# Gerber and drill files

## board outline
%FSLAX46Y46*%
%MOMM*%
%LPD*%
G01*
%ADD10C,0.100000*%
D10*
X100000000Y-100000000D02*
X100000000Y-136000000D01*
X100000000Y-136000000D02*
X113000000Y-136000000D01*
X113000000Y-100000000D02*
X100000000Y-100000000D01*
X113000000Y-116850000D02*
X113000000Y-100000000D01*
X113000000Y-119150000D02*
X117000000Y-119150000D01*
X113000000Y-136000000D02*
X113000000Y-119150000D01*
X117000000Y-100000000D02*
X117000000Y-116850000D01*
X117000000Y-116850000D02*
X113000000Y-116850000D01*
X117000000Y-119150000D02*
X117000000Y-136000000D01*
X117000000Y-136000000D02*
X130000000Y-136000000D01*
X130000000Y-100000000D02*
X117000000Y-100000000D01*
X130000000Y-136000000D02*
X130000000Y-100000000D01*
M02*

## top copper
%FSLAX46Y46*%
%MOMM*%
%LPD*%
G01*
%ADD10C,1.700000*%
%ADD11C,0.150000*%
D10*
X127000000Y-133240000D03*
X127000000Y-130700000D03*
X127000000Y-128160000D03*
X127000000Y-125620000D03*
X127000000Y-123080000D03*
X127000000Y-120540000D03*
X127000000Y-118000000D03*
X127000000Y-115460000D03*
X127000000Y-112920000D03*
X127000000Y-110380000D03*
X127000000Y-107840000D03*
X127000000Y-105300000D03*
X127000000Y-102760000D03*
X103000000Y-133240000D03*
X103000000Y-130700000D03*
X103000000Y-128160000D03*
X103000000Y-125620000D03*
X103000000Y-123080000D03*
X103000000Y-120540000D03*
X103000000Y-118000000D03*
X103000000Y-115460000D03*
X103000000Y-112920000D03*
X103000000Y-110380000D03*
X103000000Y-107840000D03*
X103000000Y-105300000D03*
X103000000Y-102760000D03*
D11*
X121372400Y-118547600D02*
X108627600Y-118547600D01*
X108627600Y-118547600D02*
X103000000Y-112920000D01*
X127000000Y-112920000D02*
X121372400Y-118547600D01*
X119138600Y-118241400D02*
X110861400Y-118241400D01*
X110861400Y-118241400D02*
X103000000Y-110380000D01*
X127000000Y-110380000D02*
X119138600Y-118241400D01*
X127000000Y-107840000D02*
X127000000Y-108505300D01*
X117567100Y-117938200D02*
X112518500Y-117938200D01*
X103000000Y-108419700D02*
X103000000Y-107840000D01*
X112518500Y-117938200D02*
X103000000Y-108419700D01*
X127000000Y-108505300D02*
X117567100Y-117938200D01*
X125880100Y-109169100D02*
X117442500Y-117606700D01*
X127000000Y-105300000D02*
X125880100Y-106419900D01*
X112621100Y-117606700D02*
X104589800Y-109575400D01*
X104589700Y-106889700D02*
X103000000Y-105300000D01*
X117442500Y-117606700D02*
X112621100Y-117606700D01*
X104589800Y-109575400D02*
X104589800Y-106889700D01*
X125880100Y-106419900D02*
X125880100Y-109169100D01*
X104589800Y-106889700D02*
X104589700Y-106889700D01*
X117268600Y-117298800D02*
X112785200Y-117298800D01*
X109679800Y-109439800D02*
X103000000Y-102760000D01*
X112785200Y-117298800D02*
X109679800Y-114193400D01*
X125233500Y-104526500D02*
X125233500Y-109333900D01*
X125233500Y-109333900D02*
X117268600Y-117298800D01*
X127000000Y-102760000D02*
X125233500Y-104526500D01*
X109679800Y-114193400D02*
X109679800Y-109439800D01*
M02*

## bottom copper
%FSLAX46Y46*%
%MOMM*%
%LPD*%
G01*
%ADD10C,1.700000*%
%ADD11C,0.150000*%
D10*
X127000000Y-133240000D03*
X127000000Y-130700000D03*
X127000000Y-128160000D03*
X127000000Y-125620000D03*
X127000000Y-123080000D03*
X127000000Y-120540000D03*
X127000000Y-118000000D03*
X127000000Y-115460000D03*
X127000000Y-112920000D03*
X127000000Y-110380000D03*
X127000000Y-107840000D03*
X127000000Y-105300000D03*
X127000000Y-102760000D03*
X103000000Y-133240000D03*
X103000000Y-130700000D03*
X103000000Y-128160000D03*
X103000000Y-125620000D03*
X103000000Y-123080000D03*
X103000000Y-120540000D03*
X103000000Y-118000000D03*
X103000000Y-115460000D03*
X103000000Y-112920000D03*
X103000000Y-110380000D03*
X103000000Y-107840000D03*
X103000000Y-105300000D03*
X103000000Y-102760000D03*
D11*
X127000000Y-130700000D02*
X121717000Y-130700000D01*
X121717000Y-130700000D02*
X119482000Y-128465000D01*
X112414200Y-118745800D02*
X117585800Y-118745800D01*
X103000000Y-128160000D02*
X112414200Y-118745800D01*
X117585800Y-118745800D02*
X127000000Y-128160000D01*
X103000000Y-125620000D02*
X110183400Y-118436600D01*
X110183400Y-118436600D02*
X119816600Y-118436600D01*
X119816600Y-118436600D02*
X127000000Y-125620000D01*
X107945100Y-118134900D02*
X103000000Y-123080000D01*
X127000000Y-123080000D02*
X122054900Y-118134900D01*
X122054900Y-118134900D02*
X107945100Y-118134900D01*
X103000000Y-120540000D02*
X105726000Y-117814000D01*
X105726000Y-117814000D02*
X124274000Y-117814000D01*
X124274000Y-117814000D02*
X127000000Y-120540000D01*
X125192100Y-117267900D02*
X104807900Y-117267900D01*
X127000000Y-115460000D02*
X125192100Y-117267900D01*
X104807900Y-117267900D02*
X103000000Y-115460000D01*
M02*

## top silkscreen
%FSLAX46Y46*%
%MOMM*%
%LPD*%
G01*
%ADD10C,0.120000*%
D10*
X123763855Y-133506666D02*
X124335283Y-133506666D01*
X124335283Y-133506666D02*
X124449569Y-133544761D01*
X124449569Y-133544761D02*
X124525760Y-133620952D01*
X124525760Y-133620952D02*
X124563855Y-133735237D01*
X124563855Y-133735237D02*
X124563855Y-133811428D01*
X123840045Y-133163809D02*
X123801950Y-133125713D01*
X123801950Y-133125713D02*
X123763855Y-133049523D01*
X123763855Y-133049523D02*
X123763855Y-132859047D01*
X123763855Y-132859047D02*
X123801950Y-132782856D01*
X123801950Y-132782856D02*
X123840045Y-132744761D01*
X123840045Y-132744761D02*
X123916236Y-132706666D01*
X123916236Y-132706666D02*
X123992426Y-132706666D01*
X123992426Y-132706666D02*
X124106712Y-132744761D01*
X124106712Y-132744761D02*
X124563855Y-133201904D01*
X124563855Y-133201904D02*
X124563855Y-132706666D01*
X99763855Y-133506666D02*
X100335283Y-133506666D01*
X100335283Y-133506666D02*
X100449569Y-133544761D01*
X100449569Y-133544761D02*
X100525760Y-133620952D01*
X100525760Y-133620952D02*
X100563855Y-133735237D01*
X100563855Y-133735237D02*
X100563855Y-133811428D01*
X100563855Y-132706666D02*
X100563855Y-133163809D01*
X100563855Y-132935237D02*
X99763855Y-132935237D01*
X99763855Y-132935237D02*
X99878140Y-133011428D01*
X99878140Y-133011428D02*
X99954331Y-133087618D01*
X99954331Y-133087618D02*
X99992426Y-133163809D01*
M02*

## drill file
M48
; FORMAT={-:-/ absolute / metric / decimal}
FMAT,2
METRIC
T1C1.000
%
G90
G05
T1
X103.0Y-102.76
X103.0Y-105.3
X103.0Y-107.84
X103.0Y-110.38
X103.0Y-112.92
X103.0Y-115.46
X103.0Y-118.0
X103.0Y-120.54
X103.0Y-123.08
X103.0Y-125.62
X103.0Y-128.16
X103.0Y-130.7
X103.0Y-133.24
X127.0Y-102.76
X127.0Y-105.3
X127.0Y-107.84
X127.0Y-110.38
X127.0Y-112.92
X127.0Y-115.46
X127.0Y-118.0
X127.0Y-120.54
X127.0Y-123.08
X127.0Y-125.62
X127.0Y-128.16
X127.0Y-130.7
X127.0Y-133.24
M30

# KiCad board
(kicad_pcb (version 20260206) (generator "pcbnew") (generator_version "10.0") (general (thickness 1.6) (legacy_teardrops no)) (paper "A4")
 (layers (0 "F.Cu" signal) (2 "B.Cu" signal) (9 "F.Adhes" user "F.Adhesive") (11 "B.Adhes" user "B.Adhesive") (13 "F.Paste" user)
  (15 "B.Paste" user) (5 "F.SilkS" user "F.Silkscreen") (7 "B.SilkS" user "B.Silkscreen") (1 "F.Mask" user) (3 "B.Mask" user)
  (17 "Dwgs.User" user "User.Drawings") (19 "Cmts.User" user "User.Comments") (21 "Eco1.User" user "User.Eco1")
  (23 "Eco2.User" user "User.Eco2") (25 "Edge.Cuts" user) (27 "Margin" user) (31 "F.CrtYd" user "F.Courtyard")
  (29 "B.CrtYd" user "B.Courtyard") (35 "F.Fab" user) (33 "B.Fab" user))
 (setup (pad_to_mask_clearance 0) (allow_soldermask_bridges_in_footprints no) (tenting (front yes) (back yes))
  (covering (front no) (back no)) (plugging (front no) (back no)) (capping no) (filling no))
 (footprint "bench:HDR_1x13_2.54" (layer "F.Cu") (at 127 133.24 90)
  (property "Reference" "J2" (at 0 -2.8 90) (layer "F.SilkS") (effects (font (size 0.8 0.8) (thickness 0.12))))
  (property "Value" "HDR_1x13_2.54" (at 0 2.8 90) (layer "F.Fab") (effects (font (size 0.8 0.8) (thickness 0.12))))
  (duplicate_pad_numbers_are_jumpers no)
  (pad "1" thru_hole circle (at 0 0 90) (size 1.7 1.7) (drill 1) (layers "*.Cu" "*.Mask") (remove_unused_layers no) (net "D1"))
  (pad "2" thru_hole circle (at 2.54 0 90) (size 1.7 1.7) (drill 1) (layers "*.Cu" "*.Mask") (remove_unused_layers no) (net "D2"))
  (pad "3" thru_hole circle (at 5.08 0 90) (size 1.7 1.7) (drill 1) (layers "*.Cu" "*.Mask") (remove_unused_layers no) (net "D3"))
  (pad "4" thru_hole circle (at 7.62 0 90) (size 1.7 1.7) (drill 1) (layers "*.Cu" "*.Mask") (remove_unused_layers no) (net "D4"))
  (pad "5" thru_hole circle (at 10.16 0 90) (size 1.7 1.7) (drill 1) (layers "*.Cu" "*.Mask") (remove_unused_layers no) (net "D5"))
  (pad "6" thru_hole circle (at 12.7 0 90) (size 1.7 1.7) (drill 1) (layers "*.Cu" "*.Mask") (remove_unused_layers no) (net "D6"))
  (pad "7" thru_hole circle (at 15.24 0 90) (size 1.7 1.7) (drill 1) (layers "*.Cu" "*.Mask") (remove_unused_layers no) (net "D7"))
  (pad "8" thru_hole circle (at 17.78 0 90) (size 1.7 1.7) (drill 1) (layers "*.Cu" "*.Mask") (remove_unused_layers no) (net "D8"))
  (pad "9" thru_hole circle (at 20.32 0 90) (size 1.7 1.7) (drill 1) (layers "*.Cu" "*.Mask") (remove_unused_layers no) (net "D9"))
  (pad "10" thru_hole circle (at 22.86 0 90) (size 1.7 1.7) (drill 1) (layers "*.Cu" "*.Mask") (remove_unused_layers no) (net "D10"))
  (pad "11" thru_hole circle (at 25.4 0 90) (size 1.7 1.7) (drill 1) (layers "*.Cu" "*.Mask") (remove_unused_layers no) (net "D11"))
  (pad "12" thru_hole circle (at 27.94 0 90) (size 1.7 1.7) (drill 1) (layers "*.Cu" "*.Mask") (remove_unused_layers no) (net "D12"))
  (pad "13" thru_hole circle (at 30.48 0 90) (size 1.7 1.7) (drill 1) (layers "*.Cu" "*.Mask") (remove_unused_layers no) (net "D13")))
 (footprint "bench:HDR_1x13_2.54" (layer "F.Cu") (at 103 133.24 90)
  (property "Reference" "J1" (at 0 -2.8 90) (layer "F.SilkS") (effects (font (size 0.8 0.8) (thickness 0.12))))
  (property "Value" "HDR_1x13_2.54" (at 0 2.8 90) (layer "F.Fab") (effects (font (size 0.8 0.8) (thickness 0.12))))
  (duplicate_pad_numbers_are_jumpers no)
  (pad "1" thru_hole circle (at 0 0 90) (size 1.7 1.7) (drill 1) (layers "*.Cu" "*.Mask") (remove_unused_layers no) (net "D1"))
  (pad "2" thru_hole circle (at 2.54 0 90) (size 1.7 1.7) (drill 1) (layers "*.Cu" "*.Mask") (remove_unused_layers no) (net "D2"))
  (pad "3" thru_hole circle (at 5.08 0 90) (size 1.7 1.7) (drill 1) (layers "*.Cu" "*.Mask") (remove_unused_layers no) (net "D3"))
  (pad "4" thru_hole circle (at 7.62 0 90) (size 1.7 1.7) (drill 1) (layers "*.Cu" "*.Mask") (remove_unused_layers no) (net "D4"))
  (pad "5" thru_hole circle (at 10.16 0 90) (size 1.7 1.7) (drill 1) (layers "*.Cu" "*.Mask") (remove_unused_layers no) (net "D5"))
  (pad "6" thru_hole circle (at 12.7 0 90) (size 1.7 1.7) (drill 1) (layers "*.Cu" "*.Mask") (remove_unused_layers no) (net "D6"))
  (pad "7" thru_hole circle (at 15.24 0 90) (size 1.7 1.7) (drill 1) (layers "*.Cu" "*.Mask") (remove_unused_layers no) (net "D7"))
  (pad "8" thru_hole circle (at 17.78 0 90) (size 1.7 1.7) (drill 1) (layers "*.Cu" "*.Mask") (remove_unused_layers no) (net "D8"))
  (pad "9" thru_hole circle (at 20.32 0 90) (size 1.7 1.7) (drill 1) (layers "*.Cu" "*.Mask") (remove_unused_layers no) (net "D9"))
  (pad "10" thru_hole circle (at 22.86 0 90) (size 1.7 1.7) (drill 1) (layers "*.Cu" "*.Mask") (remove_unused_layers no) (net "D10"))
  (pad "11" thru_hole circle (at 25.4 0 90) (size 1.7 1.7) (drill 1) (layers "*.Cu" "*.Mask") (remove_unused_layers no) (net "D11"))
  (pad "12" thru_hole circle (at 27.94 0 90) (size 1.7 1.7) (drill 1) (layers "*.Cu" "*.Mask") (remove_unused_layers no) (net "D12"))
  (pad "13" thru_hole circle (at 30.48 0 90) (size 1.7 1.7) (drill 1) (layers "*.Cu" "*.Mask") (remove_unused_layers no) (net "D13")))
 (gr_line (start 100 100) (end 100 136) (stroke (width 0.1) (type solid)) (layer "Edge.Cuts"))
 (gr_line (start 100 136) (end 113 136) (stroke (width 0.1) (type solid)) (layer "Edge.Cuts"))
 (gr_line (start 113 100) (end 100 100) (stroke (width 0.1) (type solid)) (layer "Edge.Cuts"))
 (gr_line (start 113 116.85) (end 113 100) (stroke (width 0.1) (type solid)) (layer "Edge.Cuts"))
 (gr_line (start 113 119.15) (end 117 119.15) (stroke (width 0.1) (type solid)) (layer "Edge.Cuts"))
 (gr_line (start 113 136) (end 113 119.15) (stroke (width 0.1) (type solid)) (layer "Edge.Cuts"))
 (gr_line (start 117 100) (end 117 116.85) (stroke (width 0.1) (type solid)) (layer "Edge.Cuts"))
 (gr_line (start 117 116.85) (end 113 116.85) (stroke (width 0.1) (type solid)) (layer "Edge.Cuts"))
 (gr_line (start 117 119.15) (end 117 136) (stroke (width 0.1) (type solid)) (layer "Edge.Cuts"))
 (gr_line (start 117 136) (end 130 136) (stroke (width 0.1) (type solid)) (layer "Edge.Cuts"))
 (gr_line (start 130 100) (end 117 100) (stroke (width 0.1) (type solid)) (layer "Edge.Cuts"))
 (gr_line (start 130 136) (end 130 100) (stroke (width 0.1) (type solid)) (layer "Edge.Cuts"))
 (segment (start 127 130.7) (end 121.717 130.7) (width 0.15) (layer "B.Cu") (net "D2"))
 (segment (start 121.717 130.7) (end 119.482 128.465) (width 0.15) (layer "B.Cu") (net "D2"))
 (segment (start 112.4142 118.7458) (end 117.5858 118.7458) (width 0.15) (layer "B.Cu") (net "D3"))
 (segment (start 103 128.16) (end 112.4142 118.7458) (width 0.15) (layer "B.Cu") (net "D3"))
 (segment (start 117.5858 118.7458) (end 127 128.16) (width 0.15) (layer "B.Cu") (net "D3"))
 (segment (start 103 125.62) (end 110.1834 118.4366) (width 0.15) (layer "B.Cu") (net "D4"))
 (segment (start 110.1834 118.4366) (end 119.8166 118.4366) (width 0.15) (layer "B.Cu") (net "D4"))
 (segment (start 119.8166 118.4366) (end 127 125.62) (width 0.15) (layer "B.Cu") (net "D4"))
 (segment (start 107.9451 118.1349) (end 103 123.08) (width 0.15) (layer "B.Cu") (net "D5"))
 (segment (start 127 123.08) (end 122.0549 118.1349) (width 0.15) (layer "B.Cu") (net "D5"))
 (segment (start 122.0549 118.1349) (end 107.9451 118.1349) (width 0.15) (layer "B.Cu") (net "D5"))
 (segment (start 103 120.54) (end 105.726 117.814) (width 0.15) (layer "B.Cu") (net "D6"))
 (segment (start 105.726 117.814) (end 124.274 117.814) (width 0.15) (layer "B.Cu") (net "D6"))
 (segment (start 124.274 117.814) (end 127 120.54) (width 0.15) (layer "B.Cu") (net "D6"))
 (segment (start 125.1921 117.2679) (end 104.8079 117.2679) (width 0.15) (layer "B.Cu") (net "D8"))
 (segment (start 127 115.46) (end 125.1921 117.2679) (width 0.15) (layer "B.Cu") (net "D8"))
 (segment (start 104.8079 117.2679) (end 103 115.46) (width 0.15) (layer "B.Cu") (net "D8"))
 (segment (start 121.3724 118.5476) (end 108.6276 118.5476) (width 0.15) (layer "F.Cu") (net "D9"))
 (segment (start 108.6276 118.5476) (end 103 112.92) (width 0.15) (layer "F.Cu") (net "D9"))
 (segment (start 127 112.92) (end 121.3724 118.5476) (width 0.15) (layer "F.Cu") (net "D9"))
 (segment (start 119.1386 118.2414) (end 110.8614 118.2414) (width 0.15) (layer "F.Cu") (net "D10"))
 (segment (start 110.8614 118.2414) (end 103 110.38) (width 0.15) (layer "F.Cu") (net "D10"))
 (segment (start 127 110.38) (end 119.1386 118.2414) (width 0.15) (layer "F.Cu") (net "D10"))
 (segment (start 127 107.84) (end 127 108.5053) (width 0.15) (layer "F.Cu") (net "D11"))
 (segment (start 117.5671 117.9382) (end 112.5185 117.9382) (width 0.15) (layer "F.Cu") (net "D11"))
 (segment (start 103 108.4197) (end 103 107.84) (width 0.15) (layer "F.Cu") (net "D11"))
 (segment (start 112.5185 117.9382) (end 103 108.4197) (width 0.15) (layer "F.Cu") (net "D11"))
 (segment (start 127 108.5053) (end 117.5671 117.9382) (width 0.15) (layer "F.Cu") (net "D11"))
 (segment (start 125.8801 109.1691) (end 117.4425 117.6067) (width 0.15) (layer "F.Cu") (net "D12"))
 (segment (start 127 105.3) (end 125.8801 106.4199) (width 0.15) (layer "F.Cu") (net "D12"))
 (segment (start 112.6211 117.6067) (end 104.5898 109.5754) (width 0.15) (layer "F.Cu") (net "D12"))
 (segment (start 104.5897 106.8897) (end 103 105.3) (width 0.15) (layer "F.Cu") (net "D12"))
 (segment (start 117.4425 117.6067) (end 112.6211 117.6067) (width 0.15) (layer "F.Cu") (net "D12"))
 (segment (start 104.5898 109.5754) (end 104.5898 106.8897) (width 0.15) (layer "F.Cu") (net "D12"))
 (segment (start 125.8801 106.4199) (end 125.8801 109.1691) (width 0.15) (layer "F.Cu") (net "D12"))
 (segment (start 104.5898 106.8897) (end 104.5897 106.8897) (width 0.15) (layer "F.Cu") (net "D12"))
 (segment (start 117.2686 117.2988) (end 112.7852 117.2988) (width 0.15) (layer "F.Cu") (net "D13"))
 (segment (start 109.6798 109.4398) (end 103 102.76) (width 0.15) (layer "F.Cu") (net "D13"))
 (segment (start 112.7852 117.2988) (end 109.6798 114.1934) (width 0.15) (layer "F.Cu") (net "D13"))
 (segment (start 125.2335 104.5265) (end 125.2335 109.3339) (width 0.15) (layer "F.Cu") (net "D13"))
 (segment (start 125.2335 109.3339) (end 117.2686 117.2988) (width 0.15) (layer "F.Cu") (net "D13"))
 (segment (start 127 102.76) (end 125.2335 104.5265) (width 0.15) (layer "F.Cu") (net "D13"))
 (segment (start 109.6798 114.1934) (end 109.6798 109.4398) (width 0.15) (layer "F.Cu") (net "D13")))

